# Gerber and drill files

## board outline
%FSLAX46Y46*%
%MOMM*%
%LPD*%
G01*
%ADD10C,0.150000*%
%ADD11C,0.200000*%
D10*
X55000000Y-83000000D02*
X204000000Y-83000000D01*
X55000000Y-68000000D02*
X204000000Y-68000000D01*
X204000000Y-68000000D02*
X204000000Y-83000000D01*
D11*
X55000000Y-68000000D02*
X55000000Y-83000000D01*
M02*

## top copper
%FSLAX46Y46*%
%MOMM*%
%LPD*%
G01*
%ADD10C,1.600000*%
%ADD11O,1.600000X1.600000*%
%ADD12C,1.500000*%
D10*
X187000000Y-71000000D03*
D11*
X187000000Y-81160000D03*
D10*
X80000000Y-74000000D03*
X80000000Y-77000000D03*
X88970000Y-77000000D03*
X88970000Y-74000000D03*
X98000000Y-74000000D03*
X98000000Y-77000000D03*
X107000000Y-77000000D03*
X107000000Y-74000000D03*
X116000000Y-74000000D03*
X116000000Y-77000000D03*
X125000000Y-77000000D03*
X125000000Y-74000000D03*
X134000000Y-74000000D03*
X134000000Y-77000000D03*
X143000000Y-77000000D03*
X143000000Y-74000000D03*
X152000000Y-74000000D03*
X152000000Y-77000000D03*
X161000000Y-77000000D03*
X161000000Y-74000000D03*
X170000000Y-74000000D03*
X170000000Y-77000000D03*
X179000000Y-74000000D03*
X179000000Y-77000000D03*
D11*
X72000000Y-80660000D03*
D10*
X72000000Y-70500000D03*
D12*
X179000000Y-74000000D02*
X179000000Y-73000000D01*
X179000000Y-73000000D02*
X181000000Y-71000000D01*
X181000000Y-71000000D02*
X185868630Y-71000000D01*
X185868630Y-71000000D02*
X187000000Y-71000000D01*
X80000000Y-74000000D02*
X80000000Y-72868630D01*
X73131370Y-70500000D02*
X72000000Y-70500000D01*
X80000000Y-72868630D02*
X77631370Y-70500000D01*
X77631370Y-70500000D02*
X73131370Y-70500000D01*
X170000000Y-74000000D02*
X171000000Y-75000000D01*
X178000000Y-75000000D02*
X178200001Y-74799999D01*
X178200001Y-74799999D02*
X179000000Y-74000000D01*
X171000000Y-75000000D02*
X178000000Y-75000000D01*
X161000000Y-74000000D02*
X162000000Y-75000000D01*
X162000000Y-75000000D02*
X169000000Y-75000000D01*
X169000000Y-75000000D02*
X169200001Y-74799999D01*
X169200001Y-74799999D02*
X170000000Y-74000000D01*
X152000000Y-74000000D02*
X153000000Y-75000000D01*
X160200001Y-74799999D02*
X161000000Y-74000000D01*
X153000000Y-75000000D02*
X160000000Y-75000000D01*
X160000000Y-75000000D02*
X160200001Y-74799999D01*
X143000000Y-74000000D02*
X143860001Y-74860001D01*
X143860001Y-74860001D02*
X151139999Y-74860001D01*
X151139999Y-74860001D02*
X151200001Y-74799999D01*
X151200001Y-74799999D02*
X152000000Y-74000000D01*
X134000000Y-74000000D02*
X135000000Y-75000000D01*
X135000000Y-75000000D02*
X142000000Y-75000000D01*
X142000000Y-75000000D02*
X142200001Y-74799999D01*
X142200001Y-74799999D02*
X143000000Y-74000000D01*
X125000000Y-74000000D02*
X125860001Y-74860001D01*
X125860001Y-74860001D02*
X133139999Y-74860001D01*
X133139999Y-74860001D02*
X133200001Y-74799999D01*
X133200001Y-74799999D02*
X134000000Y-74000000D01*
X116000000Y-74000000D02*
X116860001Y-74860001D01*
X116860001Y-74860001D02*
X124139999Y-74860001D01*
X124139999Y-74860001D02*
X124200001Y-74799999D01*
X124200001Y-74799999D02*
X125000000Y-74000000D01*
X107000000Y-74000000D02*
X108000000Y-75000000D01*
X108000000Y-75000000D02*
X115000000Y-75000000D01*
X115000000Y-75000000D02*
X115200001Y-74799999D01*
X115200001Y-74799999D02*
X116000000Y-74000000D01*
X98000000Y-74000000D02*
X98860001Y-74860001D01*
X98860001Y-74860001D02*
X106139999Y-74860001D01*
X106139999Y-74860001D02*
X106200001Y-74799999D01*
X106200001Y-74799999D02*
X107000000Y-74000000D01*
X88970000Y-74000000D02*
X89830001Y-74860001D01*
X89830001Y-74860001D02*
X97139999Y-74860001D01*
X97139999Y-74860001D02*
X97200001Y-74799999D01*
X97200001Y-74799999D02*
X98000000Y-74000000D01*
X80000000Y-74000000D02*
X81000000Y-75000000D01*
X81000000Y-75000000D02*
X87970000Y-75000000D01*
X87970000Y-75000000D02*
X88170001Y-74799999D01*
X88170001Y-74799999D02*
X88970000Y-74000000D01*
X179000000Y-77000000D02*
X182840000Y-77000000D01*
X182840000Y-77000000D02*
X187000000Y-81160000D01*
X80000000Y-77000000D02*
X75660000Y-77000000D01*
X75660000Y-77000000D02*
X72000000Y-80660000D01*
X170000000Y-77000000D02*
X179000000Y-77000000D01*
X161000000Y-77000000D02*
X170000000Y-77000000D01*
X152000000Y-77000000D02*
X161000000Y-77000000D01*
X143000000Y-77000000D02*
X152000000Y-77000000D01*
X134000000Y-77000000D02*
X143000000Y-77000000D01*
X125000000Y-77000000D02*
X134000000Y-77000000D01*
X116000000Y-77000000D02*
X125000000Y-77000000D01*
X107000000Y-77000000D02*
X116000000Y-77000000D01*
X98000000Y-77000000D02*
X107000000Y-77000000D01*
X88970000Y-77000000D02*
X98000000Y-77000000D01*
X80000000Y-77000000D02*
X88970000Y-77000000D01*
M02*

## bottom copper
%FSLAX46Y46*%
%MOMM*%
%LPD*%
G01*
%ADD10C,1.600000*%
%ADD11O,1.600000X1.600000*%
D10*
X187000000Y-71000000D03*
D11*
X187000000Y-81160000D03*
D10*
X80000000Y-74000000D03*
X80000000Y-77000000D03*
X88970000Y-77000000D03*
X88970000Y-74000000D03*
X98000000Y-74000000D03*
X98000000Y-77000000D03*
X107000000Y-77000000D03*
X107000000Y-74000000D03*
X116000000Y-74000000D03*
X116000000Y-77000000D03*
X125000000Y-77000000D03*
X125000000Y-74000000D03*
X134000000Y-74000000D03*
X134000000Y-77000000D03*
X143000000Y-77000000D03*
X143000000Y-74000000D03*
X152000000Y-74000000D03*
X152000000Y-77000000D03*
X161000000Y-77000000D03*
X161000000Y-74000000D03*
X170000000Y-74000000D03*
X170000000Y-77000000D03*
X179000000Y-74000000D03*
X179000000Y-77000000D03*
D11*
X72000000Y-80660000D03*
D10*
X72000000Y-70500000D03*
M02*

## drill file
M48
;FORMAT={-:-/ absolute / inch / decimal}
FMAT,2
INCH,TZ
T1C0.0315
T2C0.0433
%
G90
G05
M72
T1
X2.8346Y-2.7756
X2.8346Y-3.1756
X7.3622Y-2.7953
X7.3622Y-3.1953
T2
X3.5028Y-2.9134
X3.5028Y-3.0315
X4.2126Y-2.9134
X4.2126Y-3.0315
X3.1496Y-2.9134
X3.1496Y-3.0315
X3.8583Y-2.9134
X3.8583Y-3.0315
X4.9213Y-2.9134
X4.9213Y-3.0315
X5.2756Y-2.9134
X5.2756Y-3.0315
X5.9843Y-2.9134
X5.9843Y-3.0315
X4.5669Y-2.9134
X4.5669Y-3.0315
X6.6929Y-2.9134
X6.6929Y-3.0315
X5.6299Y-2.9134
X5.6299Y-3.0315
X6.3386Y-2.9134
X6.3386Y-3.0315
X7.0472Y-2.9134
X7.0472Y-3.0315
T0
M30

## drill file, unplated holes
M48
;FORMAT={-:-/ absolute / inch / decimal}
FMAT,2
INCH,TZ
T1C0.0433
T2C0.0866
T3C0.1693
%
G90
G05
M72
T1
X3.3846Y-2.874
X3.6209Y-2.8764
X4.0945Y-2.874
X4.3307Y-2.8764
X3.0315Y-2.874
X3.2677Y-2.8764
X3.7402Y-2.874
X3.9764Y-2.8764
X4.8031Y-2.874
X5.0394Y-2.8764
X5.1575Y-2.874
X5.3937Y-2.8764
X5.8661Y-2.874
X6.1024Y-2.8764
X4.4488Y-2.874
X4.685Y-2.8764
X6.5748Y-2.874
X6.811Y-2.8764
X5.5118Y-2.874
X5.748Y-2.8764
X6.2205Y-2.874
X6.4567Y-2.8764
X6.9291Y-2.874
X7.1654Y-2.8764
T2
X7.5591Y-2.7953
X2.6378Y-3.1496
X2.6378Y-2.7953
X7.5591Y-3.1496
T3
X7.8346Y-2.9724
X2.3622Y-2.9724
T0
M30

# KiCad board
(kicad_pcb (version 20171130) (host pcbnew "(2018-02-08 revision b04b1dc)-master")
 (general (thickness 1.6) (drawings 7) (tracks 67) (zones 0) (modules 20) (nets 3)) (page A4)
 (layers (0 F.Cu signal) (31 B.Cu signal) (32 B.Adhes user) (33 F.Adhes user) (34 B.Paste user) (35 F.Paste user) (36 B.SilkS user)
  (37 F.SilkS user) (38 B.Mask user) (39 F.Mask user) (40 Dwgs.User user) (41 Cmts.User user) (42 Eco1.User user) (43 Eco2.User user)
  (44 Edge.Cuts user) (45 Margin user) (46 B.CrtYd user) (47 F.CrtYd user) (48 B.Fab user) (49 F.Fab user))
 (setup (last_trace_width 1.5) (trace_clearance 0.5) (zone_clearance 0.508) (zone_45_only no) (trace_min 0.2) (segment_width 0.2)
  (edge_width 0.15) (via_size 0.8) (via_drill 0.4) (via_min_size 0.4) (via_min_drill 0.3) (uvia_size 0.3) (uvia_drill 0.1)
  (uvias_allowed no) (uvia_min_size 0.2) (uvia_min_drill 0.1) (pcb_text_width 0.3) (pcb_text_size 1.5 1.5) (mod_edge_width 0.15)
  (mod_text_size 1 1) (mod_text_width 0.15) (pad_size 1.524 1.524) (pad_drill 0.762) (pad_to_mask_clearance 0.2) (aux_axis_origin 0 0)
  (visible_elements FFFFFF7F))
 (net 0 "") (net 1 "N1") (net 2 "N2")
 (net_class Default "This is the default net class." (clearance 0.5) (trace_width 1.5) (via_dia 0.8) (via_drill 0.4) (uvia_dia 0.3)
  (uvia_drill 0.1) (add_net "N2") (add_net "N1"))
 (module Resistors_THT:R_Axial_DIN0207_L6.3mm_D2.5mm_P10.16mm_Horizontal (layer F.Cu) (at 187 71 270)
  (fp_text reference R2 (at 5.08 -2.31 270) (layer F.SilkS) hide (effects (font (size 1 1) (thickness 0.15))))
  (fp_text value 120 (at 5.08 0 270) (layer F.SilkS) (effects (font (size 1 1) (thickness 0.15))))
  (pad 1 thru_hole circle (at 0 0 270) (size 1.6 1.6) (drill 0.8) (layers *.Cu *.Mask) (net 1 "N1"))
  (pad 2 thru_hole oval (at 10.16 0 270) (size 1.6 1.6) (drill 0.8) (layers *.Cu *.Mask) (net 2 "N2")))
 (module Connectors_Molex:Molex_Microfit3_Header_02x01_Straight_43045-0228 (layer F.Cu) (at 80 77)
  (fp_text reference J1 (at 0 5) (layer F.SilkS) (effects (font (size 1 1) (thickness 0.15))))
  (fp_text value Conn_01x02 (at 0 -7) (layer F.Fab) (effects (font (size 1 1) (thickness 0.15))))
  (pad "" np_thru_hole circle (at 3 -3.94) (size 1.1 1.1) (drill 1.1) (layers *.Cu *.Mask))
  (pad 2 thru_hole circle (at 0 -3) (size 1.6 1.6) (drill 1.1) (layers *.Cu *.Mask) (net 1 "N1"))
  (pad 1 thru_hole circle (at 0 0) (size 1.6 1.6) (drill 1.1) (layers *.Cu *.Mask) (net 2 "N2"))
  (pad "" np_thru_hole circle (at -3 -4) (size 1.1 1.1) (drill 1.1) (layers *.Cu *.Mask)))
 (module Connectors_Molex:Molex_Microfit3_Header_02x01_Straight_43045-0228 (layer F.Cu) (at 88.97 77)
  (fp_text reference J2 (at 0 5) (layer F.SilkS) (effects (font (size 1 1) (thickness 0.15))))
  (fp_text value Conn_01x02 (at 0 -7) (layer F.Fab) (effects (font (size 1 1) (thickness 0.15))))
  (pad "" np_thru_hole circle (at -3 -4) (size 1.1 1.1) (drill 1.1) (layers *.Cu *.Mask))
  (pad 1 thru_hole circle (at 0 0) (size 1.6 1.6) (drill 1.1) (layers *.Cu *.Mask) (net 2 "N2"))
  (pad 2 thru_hole circle (at 0 -3) (size 1.6 1.6) (drill 1.1) (layers *.Cu *.Mask) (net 1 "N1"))
  (pad "" np_thru_hole circle (at 3 -3.94) (size 1.1 1.1) (drill 1.1) (layers *.Cu *.Mask)))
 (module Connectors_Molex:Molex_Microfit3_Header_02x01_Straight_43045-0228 (layer F.Cu) (at 98 77)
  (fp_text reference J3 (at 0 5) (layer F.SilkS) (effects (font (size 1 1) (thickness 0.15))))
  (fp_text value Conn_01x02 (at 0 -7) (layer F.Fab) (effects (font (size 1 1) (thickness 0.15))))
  (pad "" np_thru_hole circle (at 3 -3.94) (size 1.1 1.1) (drill 1.1) (layers *.Cu *.Mask))
  (pad 2 thru_hole circle (at 0 -3) (size 1.6 1.6) (drill 1.1) (layers *.Cu *.Mask) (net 1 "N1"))
  (pad 1 thru_hole circle (at 0 0) (size 1.6 1.6) (drill 1.1) (layers *.Cu *.Mask) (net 2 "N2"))
  (pad "" np_thru_hole circle (at -3 -4) (size 1.1 1.1) (drill 1.1) (layers *.Cu *.Mask)))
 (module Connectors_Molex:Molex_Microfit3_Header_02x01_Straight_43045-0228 (layer F.Cu) (at 107 77)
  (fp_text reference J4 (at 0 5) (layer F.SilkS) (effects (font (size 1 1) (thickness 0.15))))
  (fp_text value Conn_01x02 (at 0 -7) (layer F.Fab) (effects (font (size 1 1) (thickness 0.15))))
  (pad "" np_thru_hole circle (at -3 -4) (size 1.1 1.1) (drill 1.1) (layers *.Cu *.Mask))
  (pad 1 thru_hole circle (at 0 0) (size 1.6 1.6) (drill 1.1) (layers *.Cu *.Mask) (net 2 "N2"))
  (pad 2 thru_hole circle (at 0 -3) (size 1.6 1.6) (drill 1.1) (layers *.Cu *.Mask) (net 1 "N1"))
  (pad "" np_thru_hole circle (at 3 -3.94) (size 1.1 1.1) (drill 1.1) (layers *.Cu *.Mask)))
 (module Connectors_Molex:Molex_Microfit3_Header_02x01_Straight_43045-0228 (layer F.Cu) (at 116 77)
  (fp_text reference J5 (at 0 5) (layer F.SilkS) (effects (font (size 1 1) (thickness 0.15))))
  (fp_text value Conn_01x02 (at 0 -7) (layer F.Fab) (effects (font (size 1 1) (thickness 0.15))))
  (pad "" np_thru_hole circle (at 3 -3.94) (size 1.1 1.1) (drill 1.1) (layers *.Cu *.Mask))
  (pad 2 thru_hole circle (at 0 -3) (size 1.6 1.6) (drill 1.1) (layers *.Cu *.Mask) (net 1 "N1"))
  (pad 1 thru_hole circle (at 0 0) (size 1.6 1.6) (drill 1.1) (layers *.Cu *.Mask) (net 2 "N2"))
  (pad "" np_thru_hole circle (at -3 -4) (size 1.1 1.1) (drill 1.1) (layers *.Cu *.Mask)))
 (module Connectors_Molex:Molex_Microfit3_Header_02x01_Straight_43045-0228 (layer F.Cu) (at 125 77)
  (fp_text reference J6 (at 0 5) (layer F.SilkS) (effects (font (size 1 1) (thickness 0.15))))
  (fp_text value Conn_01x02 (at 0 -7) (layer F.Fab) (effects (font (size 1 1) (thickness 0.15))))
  (pad "" np_thru_hole circle (at -3 -4) (size 1.1 1.1) (drill 1.1) (layers *.Cu *.Mask))
  (pad 1 thru_hole circle (at 0 0) (size 1.6 1.6) (drill 1.1) (layers *.Cu *.Mask) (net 2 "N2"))
  (pad 2 thru_hole circle (at 0 -3) (size 1.6 1.6) (drill 1.1) (layers *.Cu *.Mask) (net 1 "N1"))
  (pad "" np_thru_hole circle (at 3 -3.94) (size 1.1 1.1) (drill 1.1) (layers *.Cu *.Mask)))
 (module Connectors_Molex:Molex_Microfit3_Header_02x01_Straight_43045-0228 (layer F.Cu) (at 134 77)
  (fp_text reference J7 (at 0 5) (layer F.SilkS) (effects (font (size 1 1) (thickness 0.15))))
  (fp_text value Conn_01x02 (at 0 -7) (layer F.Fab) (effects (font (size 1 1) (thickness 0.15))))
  (pad "" np_thru_hole circle (at 3 -3.94) (size 1.1 1.1) (drill 1.1) (layers *.Cu *.Mask))
  (pad 2 thru_hole circle (at 0 -3) (size 1.6 1.6) (drill 1.1) (layers *.Cu *.Mask) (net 1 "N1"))
  (pad 1 thru_hole circle (at 0 0) (size 1.6 1.6) (drill 1.1) (layers *.Cu *.Mask) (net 2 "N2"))
  (pad "" np_thru_hole circle (at -3 -4) (size 1.1 1.1) (drill 1.1) (layers *.Cu *.Mask)))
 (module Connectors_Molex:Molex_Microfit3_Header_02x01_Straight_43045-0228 (layer F.Cu) (at 143 77)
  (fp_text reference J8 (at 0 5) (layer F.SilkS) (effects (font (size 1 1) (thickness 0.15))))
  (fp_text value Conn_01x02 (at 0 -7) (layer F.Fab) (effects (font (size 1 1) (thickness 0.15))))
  (pad "" np_thru_hole circle (at -3 -4) (size 1.1 1.1) (drill 1.1) (layers *.Cu *.Mask))
  (pad 1 thru_hole circle (at 0 0) (size 1.6 1.6) (drill 1.1) (layers *.Cu *.Mask) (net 2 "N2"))
  (pad 2 thru_hole circle (at 0 -3) (size 1.6 1.6) (drill 1.1) (layers *.Cu *.Mask) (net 1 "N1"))
  (pad "" np_thru_hole circle (at 3 -3.94) (size 1.1 1.1) (drill 1.1) (layers *.Cu *.Mask)))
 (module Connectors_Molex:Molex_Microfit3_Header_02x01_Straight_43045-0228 (layer F.Cu) (at 152 77)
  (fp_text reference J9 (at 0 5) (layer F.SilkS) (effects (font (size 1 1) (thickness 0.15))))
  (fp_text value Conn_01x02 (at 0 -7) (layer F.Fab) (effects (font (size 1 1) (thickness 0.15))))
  (pad "" np_thru_hole circle (at 3 -3.94) (size 1.1 1.1) (drill 1.1) (layers *.Cu *.Mask))
  (pad 2 thru_hole circle (at 0 -3) (size 1.6 1.6) (drill 1.1) (layers *.Cu *.Mask) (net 1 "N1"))
  (pad 1 thru_hole circle (at 0 0) (size 1.6 1.6) (drill 1.1) (layers *.Cu *.Mask) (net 2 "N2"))
  (pad "" np_thru_hole circle (at -3 -4) (size 1.1 1.1) (drill 1.1) (layers *.Cu *.Mask)))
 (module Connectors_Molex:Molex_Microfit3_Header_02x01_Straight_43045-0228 (layer F.Cu) (at 161 77)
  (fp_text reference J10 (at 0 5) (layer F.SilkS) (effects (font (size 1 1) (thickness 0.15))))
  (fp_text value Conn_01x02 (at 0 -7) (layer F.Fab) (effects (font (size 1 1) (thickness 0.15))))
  (pad "" np_thru_hole circle (at -3 -4) (size 1.1 1.1) (drill 1.1) (layers *.Cu *.Mask))
  (pad 1 thru_hole circle (at 0 0) (size 1.6 1.6) (drill 1.1) (layers *.Cu *.Mask) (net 2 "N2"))
  (pad 2 thru_hole circle (at 0 -3) (size 1.6 1.6) (drill 1.1) (layers *.Cu *.Mask) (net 1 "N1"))
  (pad "" np_thru_hole circle (at 3 -3.94) (size 1.1 1.1) (drill 1.1) (layers *.Cu *.Mask)))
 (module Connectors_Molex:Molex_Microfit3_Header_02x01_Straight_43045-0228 (layer F.Cu) (at 170 77)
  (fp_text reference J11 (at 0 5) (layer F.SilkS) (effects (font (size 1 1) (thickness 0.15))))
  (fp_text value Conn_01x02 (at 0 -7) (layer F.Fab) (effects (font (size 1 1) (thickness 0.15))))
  (pad "" np_thru_hole circle (at 3 -3.94) (size 1.1 1.1) (drill 1.1) (layers *.Cu *.Mask))
  (pad 2 thru_hole circle (at 0 -3) (size 1.6 1.6) (drill 1.1) (layers *.Cu *.Mask) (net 1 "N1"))
  (pad 1 thru_hole circle (at 0 0) (size 1.6 1.6) (drill 1.1) (layers *.Cu *.Mask) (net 2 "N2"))
  (pad "" np_thru_hole circle (at -3 -4) (size 1.1 1.1) (drill 1.1) (layers *.Cu *.Mask)))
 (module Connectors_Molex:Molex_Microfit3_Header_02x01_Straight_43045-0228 (layer F.Cu) (at 179 77)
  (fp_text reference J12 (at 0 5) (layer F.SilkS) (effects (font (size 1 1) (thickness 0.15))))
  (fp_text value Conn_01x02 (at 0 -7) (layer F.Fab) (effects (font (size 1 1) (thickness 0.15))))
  (pad "" np_thru_hole circle (at 3 -3.94) (size 1.1 1.1) (drill 1.1) (layers *.Cu *.Mask))
  (pad 2 thru_hole circle (at 0 -3) (size 1.6 1.6) (drill 1.1) (layers *.Cu *.Mask) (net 1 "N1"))
  (pad 1 thru_hole circle (at 0 0) (size 1.6 1.6) (drill 1.1) (layers *.Cu *.Mask) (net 2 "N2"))
  (pad "" np_thru_hole circle (at -3 -4) (size 1.1 1.1) (drill 1.1) (layers *.Cu *.Mask)))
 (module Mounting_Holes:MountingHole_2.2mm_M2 (layer F.Cu) (at 67 71)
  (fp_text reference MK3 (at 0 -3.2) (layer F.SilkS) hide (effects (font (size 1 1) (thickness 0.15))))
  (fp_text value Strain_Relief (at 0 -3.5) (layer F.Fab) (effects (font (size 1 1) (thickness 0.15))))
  (pad 1 np_thru_hole circle (at 0 0) (size 2.2 2.2) (drill 2.2) (layers *.Cu *.Mask)))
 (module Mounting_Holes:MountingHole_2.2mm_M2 (layer F.Cu) (at 67 80)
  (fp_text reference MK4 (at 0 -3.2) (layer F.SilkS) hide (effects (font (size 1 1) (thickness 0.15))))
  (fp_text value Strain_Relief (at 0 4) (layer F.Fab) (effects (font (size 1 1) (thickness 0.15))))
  (pad 1 np_thru_hole circle (at 0 0) (size 2.2 2.2) (drill 2.2) (layers *.Cu *.Mask)))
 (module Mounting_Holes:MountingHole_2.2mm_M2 (layer F.Cu) (at 192 71)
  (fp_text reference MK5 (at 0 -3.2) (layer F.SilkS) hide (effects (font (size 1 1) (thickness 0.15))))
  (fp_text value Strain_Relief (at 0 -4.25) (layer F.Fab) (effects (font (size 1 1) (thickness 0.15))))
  (pad 1 np_thru_hole circle (at 0 0) (size 2.2 2.2) (drill 2.2) (layers *.Cu *.Mask)))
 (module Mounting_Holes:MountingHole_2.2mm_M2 (layer F.Cu) (at 192 80)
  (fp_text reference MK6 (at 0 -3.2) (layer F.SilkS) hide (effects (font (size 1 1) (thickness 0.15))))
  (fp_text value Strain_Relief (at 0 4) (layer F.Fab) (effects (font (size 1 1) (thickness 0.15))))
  (pad 1 np_thru_hole circle (at 0 0) (size 2.2 2.2) (drill 2.2) (layers *.Cu *.Mask)))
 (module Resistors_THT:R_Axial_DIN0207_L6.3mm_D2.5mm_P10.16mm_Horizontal (layer F.Cu) (at 72 70.5 270)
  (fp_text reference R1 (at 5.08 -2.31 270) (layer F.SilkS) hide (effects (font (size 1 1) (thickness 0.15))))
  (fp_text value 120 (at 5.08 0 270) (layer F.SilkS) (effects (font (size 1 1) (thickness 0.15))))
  (pad 2 thru_hole oval (at 10.16 0 270) (size 1.6 1.6) (drill 0.8) (layers *.Cu *.Mask) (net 2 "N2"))
  (pad 1 thru_hole circle (at 0 0 270) (size 1.6 1.6) (drill 0.8) (layers *.Cu *.Mask) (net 1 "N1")))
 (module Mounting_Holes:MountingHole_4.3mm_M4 (layer F.Cu) (at 60 75.5)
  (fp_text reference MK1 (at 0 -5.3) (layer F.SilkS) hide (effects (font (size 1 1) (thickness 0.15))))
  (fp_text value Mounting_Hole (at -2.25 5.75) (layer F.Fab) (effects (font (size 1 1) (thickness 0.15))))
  (pad 1 np_thru_hole circle (at 0 0) (size 4.3 4.3) (drill 4.3) (layers *.Cu *.Mask)))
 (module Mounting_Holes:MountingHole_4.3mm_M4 (layer F.Cu) (at 199 75.5)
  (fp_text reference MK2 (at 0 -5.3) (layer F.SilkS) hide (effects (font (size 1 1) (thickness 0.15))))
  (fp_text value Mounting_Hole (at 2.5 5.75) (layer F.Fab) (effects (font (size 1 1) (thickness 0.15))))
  (pad 1 np_thru_hole circle (at 0 0) (size 4.3 4.3) (drill 4.3) (layers *.Cu *.Mask)))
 (gr_line (start 55 83) (end 204 83) (layer Edge.Cuts) (width 0.15))
 (gr_line (start 55 68) (end 204 68) (layer Edge.Cuts) (width 0.15))
 (gr_line (start 204 68) (end 204 83) (layer Edge.Cuts) (width 0.15))
 (gr_line (start 55 68) (end 55 83) (layer Edge.Cuts) (width 0.2))
 (segment (start 179 74) (end 179 73) (width 1.5) (layer F.Cu) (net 1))
 (segment (start 179 73) (end 181 71) (width 1.5) (layer F.Cu) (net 1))
 (segment (start 181 71) (end 185.86863 71) (width 1.5) (layer F.Cu) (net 1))
 (segment (start 185.86863 71) (end 187 71) (width 1.5) (layer F.Cu) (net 1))
 (segment (start 80 74) (end 80 72.86863) (width 1.5) (layer F.Cu) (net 1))
 (segment (start 73.13137 70.5) (end 72 70.5) (width 1.5) (layer F.Cu) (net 1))
 (segment (start 80 72.86863) (end 77.63137 70.5) (width 1.5) (layer F.Cu) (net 1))
 (segment (start 77.63137 70.5) (end 73.13137 70.5) (width 1.5) (layer F.Cu) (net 1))
 (segment (start 170 74) (end 171 75) (width 1.5) (layer F.Cu) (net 1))
 (segment (start 178 75) (end 178.200001 74.799999) (width 1.5) (layer F.Cu) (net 1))
 (segment (start 178.200001 74.799999) (end 179 74) (width 1.5) (layer F.Cu) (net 1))
 (segment (start 171 75) (end 178 75) (width 1.5) (layer F.Cu) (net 1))
 (segment (start 161 74) (end 162 75) (width 1.5) (layer F.Cu) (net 1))
 (segment (start 162 75) (end 169 75) (width 1.5) (layer F.Cu) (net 1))
 (segment (start 169 75) (end 169.200001 74.799999) (width 1.5) (layer F.Cu) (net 1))
 (segment (start 169.200001 74.799999) (end 170 74) (width 1.5) (layer F.Cu) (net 1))
 (segment (start 152 74) (end 153 75) (width 1.5) (layer F.Cu) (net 1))
 (segment (start 160.200001 74.799999) (end 161 74) (width 1.5) (layer F.Cu) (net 1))
 (segment (start 153 75) (end 160 75) (width 1.5) (layer F.Cu) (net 1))
 (segment (start 160 75) (end 160.200001 74.799999) (width 1.5) (layer F.Cu) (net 1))
 (segment (start 143 74) (end 143.860001 74.860001) (width 1.5) (layer F.Cu) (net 1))
 (segment (start 143.860001 74.860001) (end 151.139999 74.860001) (width 1.5) (layer F.Cu) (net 1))
 (segment (start 151.139999 74.860001) (end 151.200001 74.799999) (width 1.5) (layer F.Cu) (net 1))
 (segment (start 151.200001 74.799999) (end 152 74) (width 1.5) (layer F.Cu) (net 1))
 (segment (start 134 74) (end 135 75) (width 1.5) (layer F.Cu) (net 1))
 (segment (start 135 75) (end 142 75) (width 1.5) (layer F.Cu) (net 1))
 (segment (start 142 75) (end 142.200001 74.799999) (width 1.5) (layer F.Cu) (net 1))
 (segment (start 142.200001 74.799999) (end 143 74) (width 1.5) (layer F.Cu) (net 1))
 (segment (start 125 74) (end 125.860001 74.860001) (width 1.5) (layer F.Cu) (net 1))
 (segment (start 125.860001 74.860001) (end 133.139999 74.860001) (width 1.5) (layer F.Cu) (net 1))
 (segment (start 133.139999 74.860001) (end 133.200001 74.799999) (width 1.5) (layer F.Cu) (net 1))
 (segment (start 133.200001 74.799999) (end 134 74) (width 1.5) (layer F.Cu) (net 1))
 (segment (start 116 74) (end 116.860001 74.860001) (width 1.5) (layer F.Cu) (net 1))
 (segment (start 116.860001 74.860001) (end 124.139999 74.860001) (width 1.5) (layer F.Cu) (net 1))
 (segment (start 124.139999 74.860001) (end 124.200001 74.799999) (width 1.5) (layer F.Cu) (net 1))
 (segment (start 124.200001 74.799999) (end 125 74) (width 1.5) (layer F.Cu) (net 1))
 (segment (start 107 74) (end 108 75) (width 1.5) (layer F.Cu) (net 1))
 (segment (start 108 75) (end 115 75) (width 1.5) (layer F.Cu) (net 1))
 (segment (start 115 75) (end 115.200001 74.799999) (width 1.5) (layer F.Cu) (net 1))
 (segment (start 115.200001 74.799999) (end 116 74) (width 1.5) (layer F.Cu) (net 1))
 (segment (start 98 74) (end 98.860001 74.860001) (width 1.5) (layer F.Cu) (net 1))
 (segment (start 98.860001 74.860001) (end 106.139999 74.860001) (width 1.5) (layer F.Cu) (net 1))
 (segment (start 106.139999 74.860001) (end 106.200001 74.799999) (width 1.5) (layer F.Cu) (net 1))
 (segment (start 106.200001 74.799999) (end 107 74) (width 1.5) (layer F.Cu) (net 1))
 (segment (start 88.97 74) (end 89.830001 74.860001) (width 1.5) (layer F.Cu) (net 1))
 (segment (start 89.830001 74.860001) (end 97.139999 74.860001) (width 1.5) (layer F.Cu) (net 1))
 (segment (start 97.139999 74.860001) (end 97.200001 74.799999) (width 1.5) (layer F.Cu) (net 1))
 (segment (start 97.200001 74.799999) (end 98 74) (width 1.5) (layer F.Cu) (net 1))
 (segment (start 80 74) (end 81 75) (width 1.5) (layer F.Cu) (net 1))
 (segment (start 81 75) (end 87.97 75) (width 1.5) (layer F.Cu) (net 1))
 (segment (start 87.97 75) (end 88.170001 74.799999) (width 1.5) (layer F.Cu) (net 1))
 (segment (start 88.170001 74.799999) (end 88.97 74) (width 1.5) (layer F.Cu) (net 1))
 (segment (start 179 77) (end 182.84 77) (width 1.5) (layer F.Cu) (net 2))
 (segment (start 182.84 77) (end 187 81.16) (width 1.5) (layer F.Cu) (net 2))
 (segment (start 80 77) (end 75.66 77) (width 1.5) (layer F.Cu) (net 2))
 (segment (start 75.66 77) (end 72 80.66) (width 1.5) (layer F.Cu) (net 2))
 (segment (start 170 77) (end 179 77) (width 1.5) (layer F.Cu) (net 2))
 (segment (start 161 77) (end 170 77) (width 1.5) (layer F.Cu) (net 2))
 (segment (start 152 77) (end 161 77) (width 1.5) (layer F.Cu) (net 2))
 (segment (start 143 77) (end 152 77) (width 1.5) (layer F.Cu) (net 2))
 (segment (start 134 77) (end 143 77) (width 1.5) (layer F.Cu) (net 2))
 (segment (start 125 77) (end 134 77) (width 1.5) (layer F.Cu) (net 2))
 (segment (start 116 77) (end 125 77) (width 1.5) (layer F.Cu) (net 2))
 (segment (start 107 77) (end 116 77) (width 1.5) (layer F.Cu) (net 2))
 (segment (start 98 77) (end 107 77) (width 1.5) (layer F.Cu) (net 2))
 (segment (start 88.97 77) (end 98 77) (width 1.5) (layer F.Cu) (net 2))
 (segment (start 80 77) (end 88.97 77) (width 1.5) (layer F.Cu) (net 2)))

